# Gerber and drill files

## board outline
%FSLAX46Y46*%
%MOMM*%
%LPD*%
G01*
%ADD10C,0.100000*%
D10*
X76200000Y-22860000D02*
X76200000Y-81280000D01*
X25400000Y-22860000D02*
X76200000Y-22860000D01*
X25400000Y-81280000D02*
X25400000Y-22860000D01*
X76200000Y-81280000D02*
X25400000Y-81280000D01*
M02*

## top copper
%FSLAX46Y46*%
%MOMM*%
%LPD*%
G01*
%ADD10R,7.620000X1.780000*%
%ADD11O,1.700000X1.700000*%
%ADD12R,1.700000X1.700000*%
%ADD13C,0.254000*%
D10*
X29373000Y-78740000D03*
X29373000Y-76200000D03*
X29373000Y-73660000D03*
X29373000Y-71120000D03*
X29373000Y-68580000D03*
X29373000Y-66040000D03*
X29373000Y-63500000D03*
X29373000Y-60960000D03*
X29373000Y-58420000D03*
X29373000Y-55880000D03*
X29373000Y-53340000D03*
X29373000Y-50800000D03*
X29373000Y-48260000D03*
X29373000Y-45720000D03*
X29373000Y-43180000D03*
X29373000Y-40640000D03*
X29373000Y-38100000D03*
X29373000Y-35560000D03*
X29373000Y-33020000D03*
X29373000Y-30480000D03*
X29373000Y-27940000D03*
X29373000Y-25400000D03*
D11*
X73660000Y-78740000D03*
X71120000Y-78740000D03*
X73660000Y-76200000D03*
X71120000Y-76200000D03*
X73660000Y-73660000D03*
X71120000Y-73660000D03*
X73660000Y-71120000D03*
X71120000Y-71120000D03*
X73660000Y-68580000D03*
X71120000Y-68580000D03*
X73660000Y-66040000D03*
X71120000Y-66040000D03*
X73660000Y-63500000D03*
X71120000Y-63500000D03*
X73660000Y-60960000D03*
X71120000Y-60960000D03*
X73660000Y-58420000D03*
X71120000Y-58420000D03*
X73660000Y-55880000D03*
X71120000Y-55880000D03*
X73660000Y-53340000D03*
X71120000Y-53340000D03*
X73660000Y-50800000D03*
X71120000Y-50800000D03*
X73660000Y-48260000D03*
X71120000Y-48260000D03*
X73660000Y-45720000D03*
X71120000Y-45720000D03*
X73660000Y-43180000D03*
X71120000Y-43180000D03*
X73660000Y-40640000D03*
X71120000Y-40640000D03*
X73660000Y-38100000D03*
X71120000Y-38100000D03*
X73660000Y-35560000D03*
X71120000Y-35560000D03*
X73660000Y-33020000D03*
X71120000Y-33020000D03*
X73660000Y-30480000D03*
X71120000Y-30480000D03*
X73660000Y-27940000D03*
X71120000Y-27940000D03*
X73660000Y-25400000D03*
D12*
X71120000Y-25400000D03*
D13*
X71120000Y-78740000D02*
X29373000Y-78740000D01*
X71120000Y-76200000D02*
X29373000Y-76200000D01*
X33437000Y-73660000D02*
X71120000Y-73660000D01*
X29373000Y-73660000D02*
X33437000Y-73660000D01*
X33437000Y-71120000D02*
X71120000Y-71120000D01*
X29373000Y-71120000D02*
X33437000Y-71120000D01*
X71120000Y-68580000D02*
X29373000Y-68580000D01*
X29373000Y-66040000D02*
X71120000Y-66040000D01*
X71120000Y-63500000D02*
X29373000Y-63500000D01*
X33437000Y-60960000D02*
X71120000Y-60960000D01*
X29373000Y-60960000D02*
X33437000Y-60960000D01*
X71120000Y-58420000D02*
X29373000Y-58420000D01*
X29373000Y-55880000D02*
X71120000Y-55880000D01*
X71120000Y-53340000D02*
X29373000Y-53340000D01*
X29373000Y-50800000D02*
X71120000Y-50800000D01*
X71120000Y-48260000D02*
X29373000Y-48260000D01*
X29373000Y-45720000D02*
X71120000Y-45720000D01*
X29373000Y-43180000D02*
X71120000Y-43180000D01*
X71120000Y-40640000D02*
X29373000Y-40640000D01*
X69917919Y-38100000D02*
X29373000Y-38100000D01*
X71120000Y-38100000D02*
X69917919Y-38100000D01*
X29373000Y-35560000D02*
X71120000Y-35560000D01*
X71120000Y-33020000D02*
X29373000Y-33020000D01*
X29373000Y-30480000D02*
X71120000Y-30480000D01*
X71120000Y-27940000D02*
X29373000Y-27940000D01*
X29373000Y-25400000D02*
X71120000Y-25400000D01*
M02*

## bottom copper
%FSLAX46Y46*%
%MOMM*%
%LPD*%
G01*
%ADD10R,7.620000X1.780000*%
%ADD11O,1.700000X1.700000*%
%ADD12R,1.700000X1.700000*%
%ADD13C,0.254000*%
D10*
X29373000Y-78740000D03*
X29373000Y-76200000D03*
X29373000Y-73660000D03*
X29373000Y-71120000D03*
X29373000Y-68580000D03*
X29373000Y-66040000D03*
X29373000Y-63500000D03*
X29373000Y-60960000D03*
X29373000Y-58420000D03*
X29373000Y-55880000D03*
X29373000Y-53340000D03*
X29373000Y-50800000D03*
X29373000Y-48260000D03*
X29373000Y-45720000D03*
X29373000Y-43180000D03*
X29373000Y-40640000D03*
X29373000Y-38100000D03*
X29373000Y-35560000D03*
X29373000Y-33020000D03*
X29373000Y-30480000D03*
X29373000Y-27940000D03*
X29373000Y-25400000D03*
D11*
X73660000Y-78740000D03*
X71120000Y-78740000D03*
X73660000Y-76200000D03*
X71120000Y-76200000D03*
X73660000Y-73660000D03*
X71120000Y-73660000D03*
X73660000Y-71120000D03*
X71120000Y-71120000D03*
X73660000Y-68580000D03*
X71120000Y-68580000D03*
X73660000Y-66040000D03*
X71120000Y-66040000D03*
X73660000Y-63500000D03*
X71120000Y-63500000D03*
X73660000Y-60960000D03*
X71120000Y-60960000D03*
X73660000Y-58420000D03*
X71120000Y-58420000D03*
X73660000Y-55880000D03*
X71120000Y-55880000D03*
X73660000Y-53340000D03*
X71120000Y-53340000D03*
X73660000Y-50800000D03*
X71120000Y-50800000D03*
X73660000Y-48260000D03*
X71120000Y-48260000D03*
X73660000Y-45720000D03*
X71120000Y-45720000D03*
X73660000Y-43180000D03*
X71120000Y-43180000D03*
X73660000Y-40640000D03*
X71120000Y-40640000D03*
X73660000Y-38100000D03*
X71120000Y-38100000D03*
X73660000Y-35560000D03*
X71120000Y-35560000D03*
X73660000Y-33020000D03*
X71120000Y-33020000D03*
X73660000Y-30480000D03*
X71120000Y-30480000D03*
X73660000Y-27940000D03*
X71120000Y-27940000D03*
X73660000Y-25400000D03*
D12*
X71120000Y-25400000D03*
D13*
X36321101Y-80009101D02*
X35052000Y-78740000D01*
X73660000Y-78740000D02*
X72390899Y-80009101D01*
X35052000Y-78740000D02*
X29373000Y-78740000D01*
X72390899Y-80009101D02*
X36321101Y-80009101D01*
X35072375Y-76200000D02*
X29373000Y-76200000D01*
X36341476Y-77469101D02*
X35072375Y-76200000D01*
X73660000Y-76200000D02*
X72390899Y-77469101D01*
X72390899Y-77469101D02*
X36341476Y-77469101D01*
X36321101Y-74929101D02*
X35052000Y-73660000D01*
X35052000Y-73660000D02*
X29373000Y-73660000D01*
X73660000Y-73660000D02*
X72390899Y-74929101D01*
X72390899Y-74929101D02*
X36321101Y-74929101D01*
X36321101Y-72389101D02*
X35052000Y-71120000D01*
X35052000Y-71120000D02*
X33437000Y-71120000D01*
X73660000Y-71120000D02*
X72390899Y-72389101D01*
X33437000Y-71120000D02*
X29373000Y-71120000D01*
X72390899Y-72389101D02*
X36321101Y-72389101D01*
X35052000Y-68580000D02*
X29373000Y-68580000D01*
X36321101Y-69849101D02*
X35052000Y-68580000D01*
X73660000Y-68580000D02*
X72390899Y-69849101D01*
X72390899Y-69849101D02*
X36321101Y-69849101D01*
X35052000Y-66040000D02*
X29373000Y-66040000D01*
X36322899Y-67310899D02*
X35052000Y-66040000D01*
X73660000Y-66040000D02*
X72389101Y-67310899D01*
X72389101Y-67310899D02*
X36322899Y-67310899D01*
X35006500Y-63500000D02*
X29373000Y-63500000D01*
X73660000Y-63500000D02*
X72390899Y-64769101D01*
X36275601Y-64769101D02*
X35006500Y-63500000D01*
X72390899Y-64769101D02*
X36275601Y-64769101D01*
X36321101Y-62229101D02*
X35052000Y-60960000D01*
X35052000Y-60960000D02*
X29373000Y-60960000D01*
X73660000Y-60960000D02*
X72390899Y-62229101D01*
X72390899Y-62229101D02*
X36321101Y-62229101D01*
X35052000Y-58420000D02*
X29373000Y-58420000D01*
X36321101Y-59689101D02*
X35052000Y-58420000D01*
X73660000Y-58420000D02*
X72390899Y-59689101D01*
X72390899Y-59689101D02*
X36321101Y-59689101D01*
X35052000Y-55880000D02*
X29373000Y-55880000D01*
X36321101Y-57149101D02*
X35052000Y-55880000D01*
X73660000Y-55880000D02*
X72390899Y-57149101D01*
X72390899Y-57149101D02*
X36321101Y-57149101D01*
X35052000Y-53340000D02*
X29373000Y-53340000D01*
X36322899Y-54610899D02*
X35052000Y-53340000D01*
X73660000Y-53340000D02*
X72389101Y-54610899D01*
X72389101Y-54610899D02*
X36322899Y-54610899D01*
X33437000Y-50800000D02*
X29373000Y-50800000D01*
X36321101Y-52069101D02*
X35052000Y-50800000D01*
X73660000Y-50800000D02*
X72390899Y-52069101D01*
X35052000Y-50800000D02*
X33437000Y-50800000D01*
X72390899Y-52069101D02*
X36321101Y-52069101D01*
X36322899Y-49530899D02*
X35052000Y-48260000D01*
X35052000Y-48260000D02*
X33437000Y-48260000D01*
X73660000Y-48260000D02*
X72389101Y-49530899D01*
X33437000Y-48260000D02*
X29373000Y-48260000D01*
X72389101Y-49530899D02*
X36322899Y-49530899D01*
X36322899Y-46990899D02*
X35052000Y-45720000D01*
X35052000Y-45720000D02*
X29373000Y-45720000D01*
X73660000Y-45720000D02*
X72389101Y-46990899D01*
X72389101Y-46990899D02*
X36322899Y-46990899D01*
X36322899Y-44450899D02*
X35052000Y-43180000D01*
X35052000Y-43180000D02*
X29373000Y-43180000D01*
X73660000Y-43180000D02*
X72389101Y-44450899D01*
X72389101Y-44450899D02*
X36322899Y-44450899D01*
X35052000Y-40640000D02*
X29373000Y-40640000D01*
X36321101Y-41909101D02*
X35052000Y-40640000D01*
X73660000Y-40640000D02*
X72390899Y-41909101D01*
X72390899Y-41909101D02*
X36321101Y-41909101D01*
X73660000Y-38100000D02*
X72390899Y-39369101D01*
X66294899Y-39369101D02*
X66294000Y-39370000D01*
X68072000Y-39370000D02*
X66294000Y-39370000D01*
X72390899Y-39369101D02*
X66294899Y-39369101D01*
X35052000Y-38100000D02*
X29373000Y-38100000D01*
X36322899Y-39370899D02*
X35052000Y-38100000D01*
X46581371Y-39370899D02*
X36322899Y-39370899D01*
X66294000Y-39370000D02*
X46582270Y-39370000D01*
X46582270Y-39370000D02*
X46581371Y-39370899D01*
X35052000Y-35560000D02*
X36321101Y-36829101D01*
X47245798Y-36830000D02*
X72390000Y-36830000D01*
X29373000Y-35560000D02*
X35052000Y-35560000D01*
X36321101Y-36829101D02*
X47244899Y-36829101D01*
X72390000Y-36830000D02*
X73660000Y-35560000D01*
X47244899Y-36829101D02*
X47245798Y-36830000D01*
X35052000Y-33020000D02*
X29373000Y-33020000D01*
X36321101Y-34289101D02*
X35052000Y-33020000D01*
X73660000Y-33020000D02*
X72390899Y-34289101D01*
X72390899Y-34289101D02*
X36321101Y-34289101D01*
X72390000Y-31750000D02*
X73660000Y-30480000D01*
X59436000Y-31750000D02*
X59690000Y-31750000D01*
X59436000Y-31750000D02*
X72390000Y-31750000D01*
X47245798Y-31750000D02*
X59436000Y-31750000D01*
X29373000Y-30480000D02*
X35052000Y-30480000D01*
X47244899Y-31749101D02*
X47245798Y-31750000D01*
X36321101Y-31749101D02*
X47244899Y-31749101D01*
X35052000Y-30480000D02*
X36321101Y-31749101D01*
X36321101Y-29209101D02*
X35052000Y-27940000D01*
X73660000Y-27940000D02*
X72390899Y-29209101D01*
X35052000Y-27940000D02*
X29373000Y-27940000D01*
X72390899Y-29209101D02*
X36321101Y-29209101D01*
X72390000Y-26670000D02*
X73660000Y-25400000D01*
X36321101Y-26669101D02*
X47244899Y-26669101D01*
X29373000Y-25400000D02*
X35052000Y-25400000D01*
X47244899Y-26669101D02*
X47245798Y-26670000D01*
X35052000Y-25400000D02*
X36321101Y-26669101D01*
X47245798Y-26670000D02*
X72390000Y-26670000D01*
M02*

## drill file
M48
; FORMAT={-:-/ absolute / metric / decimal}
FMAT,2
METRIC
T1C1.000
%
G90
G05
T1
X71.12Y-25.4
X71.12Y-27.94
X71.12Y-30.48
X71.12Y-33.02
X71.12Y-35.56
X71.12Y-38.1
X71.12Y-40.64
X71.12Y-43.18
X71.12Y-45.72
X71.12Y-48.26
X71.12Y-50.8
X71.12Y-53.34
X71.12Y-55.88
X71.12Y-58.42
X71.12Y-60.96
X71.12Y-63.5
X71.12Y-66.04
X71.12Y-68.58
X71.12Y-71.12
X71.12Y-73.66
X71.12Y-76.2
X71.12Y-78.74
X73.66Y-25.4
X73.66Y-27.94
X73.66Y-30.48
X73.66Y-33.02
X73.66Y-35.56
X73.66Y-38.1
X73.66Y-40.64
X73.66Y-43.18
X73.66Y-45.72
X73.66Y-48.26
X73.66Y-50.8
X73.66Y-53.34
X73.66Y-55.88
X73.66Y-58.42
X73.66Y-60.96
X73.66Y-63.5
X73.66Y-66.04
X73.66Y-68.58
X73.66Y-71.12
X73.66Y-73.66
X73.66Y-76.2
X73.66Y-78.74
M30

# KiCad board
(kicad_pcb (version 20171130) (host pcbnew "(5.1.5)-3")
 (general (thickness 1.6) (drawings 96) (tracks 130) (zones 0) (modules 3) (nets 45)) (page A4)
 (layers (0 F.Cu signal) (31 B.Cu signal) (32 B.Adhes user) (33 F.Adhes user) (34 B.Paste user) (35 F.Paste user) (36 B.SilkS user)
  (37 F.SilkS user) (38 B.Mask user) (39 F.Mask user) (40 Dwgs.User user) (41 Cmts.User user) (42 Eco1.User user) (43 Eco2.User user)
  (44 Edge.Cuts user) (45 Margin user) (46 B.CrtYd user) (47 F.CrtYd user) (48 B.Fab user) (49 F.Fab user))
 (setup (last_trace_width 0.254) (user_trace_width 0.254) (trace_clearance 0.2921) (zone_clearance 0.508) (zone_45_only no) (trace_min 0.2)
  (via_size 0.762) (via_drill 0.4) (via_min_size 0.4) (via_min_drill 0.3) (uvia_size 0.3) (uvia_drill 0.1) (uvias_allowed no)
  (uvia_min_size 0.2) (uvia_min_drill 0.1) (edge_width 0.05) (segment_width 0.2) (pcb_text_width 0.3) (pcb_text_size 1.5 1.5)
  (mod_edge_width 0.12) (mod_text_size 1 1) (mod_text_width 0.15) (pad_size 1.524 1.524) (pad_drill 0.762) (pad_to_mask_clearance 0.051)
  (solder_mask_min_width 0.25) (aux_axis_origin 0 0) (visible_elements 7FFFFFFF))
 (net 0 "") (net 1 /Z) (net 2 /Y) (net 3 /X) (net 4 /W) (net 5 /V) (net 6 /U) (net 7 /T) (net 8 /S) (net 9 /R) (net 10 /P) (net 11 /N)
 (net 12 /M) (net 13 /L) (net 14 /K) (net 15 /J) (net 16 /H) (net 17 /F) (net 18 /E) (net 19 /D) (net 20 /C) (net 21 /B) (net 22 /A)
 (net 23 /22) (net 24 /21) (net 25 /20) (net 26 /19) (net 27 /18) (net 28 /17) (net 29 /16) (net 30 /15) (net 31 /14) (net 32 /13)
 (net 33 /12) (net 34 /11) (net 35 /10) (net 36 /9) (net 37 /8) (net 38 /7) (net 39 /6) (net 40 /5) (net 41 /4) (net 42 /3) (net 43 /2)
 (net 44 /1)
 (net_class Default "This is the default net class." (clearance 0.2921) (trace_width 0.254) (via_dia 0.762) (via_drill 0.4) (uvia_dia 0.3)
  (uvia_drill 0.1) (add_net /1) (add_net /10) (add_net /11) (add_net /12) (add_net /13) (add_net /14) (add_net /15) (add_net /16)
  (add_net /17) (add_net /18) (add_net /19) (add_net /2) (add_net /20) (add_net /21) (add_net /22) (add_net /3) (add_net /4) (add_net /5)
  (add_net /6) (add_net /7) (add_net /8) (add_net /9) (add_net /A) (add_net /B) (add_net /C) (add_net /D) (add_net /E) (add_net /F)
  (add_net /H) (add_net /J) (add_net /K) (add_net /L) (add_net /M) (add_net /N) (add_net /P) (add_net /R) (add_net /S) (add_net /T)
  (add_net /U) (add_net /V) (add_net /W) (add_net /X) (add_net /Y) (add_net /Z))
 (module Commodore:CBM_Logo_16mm (layer F.Cu) (at 54.61 52.07 90)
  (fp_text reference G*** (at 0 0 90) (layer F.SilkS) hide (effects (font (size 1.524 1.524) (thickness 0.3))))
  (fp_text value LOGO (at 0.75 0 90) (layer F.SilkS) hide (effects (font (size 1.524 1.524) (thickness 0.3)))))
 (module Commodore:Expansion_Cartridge (layer F.Cu) (at 25.527 23.749 90)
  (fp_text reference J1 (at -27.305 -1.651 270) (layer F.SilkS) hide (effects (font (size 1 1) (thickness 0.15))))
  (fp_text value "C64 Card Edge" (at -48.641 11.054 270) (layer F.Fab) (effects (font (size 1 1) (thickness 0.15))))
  (pad Z connect rect (at -54.991 3.846 270) (size 1.78 7.62) (layers B.Cu B.Mask) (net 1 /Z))
  (pad Y connect rect (at -52.451 3.846 270) (size 1.78 7.62) (layers B.Cu B.Mask) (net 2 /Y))
  (pad X connect rect (at -49.911 3.846 270) (size 1.78 7.62) (layers B.Cu B.Mask) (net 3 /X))
  (pad W connect rect (at -47.371 3.846 270) (size 1.78 7.62) (layers B.Cu B.Mask) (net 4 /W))
  (pad V connect rect (at -44.831 3.846 270) (size 1.78 7.62) (layers B.Cu B.Mask) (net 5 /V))
  (pad U connect rect (at -42.291 3.846 270) (size 1.78 7.62) (layers B.Cu B.Mask) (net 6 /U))
  (pad T connect rect (at -39.751 3.846 270) (size 1.78 7.62) (layers B.Cu B.Mask) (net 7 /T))
  (pad S connect rect (at -37.211 3.846 270) (size 1.78 7.62) (layers B.Cu B.Mask) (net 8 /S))
  (pad R connect rect (at -34.671 3.846 270) (size 1.78 7.62) (layers B.Cu B.Mask) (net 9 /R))
  (pad P connect rect (at -32.131 3.846 270) (size 1.78 7.62) (layers B.Cu B.Mask) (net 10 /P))
  (pad N connect rect (at -29.591 3.846 270) (size 1.78 7.62) (layers B.Cu B.Mask) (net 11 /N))
  (pad M connect rect (at -27.051 3.846 270) (size 1.78 7.62) (layers B.Cu B.Mask) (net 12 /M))
  (pad L connect rect (at -24.511 3.846 270) (size 1.78 7.62) (layers B.Cu B.Mask) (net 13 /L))
  (pad K connect rect (at -21.971 3.846 270) (size 1.78 7.62) (layers B.Cu B.Mask) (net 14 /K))
  (pad J connect rect (at -19.431 3.846 270) (size 1.78 7.62) (layers B.Cu B.Mask) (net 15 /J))
  (pad H connect rect (at -16.891 3.846 270) (size 1.78 7.62) (layers B.Cu B.Mask) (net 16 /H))
  (pad F connect rect (at -14.351 3.846 270) (size 1.78 7.62) (layers B.Cu B.Mask) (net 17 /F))
  (pad E connect rect (at -11.811 3.846 270) (size 1.78 7.62) (layers B.Cu B.Mask) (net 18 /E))
  (pad D connect rect (at -9.271 3.846 270) (size 1.78 7.62) (layers B.Cu B.Mask) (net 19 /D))
  (pad C connect rect (at -6.731 3.846 270) (size 1.78 7.62) (layers B.Cu B.Mask) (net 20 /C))
  (pad B connect rect (at -4.191 3.846 270) (size 1.78 7.62) (layers B.Cu B.Mask) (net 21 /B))
  (pad A connect rect (at -1.651 3.846 270) (size 1.78 7.62) (layers B.Cu B.Mask) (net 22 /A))
  (pad 22 connect rect (at -54.991 3.846 270) (size 1.78 7.62) (layers F.Cu F.Mask) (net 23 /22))
  (pad 21 connect rect (at -52.451 3.846 270) (size 1.78 7.62) (layers F.Cu F.Mask) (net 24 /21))
  (pad 20 connect rect (at -49.911 3.846 270) (size 1.78 7.62) (layers F.Cu F.Mask) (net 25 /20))
  (pad 19 connect rect (at -47.371 3.846 270) (size 1.78 7.62) (layers F.Cu F.Mask) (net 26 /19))
  (pad 18 connect rect (at -44.831 3.846 270) (size 1.78 7.62) (layers F.Cu F.Mask) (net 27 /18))
  (pad 17 connect rect (at -42.291 3.846 270) (size 1.78 7.62) (layers F.Cu F.Mask) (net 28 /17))
  (pad 16 connect rect (at -39.751 3.846 270) (size 1.78 7.62) (layers F.Cu F.Mask) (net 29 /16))
  (pad 15 connect rect (at -37.211 3.846 270) (size 1.78 7.62) (layers F.Cu F.Mask) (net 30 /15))
  (pad 14 connect rect (at -34.671 3.846 270) (size 1.78 7.62) (layers F.Cu F.Mask) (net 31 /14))
  (pad 13 connect rect (at -32.131 3.846 270) (size 1.78 7.62) (layers F.Cu F.Mask) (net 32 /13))
  (pad 12 connect rect (at -29.591 3.846 270) (size 1.78 7.62) (layers F.Cu F.Mask) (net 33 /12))
  (pad 11 connect rect (at -27.051 3.846 270) (size 1.78 7.62) (layers F.Cu F.Mask) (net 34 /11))
  (pad 10 connect rect (at -24.511 3.846 270) (size 1.78 7.62) (layers F.Cu F.Mask) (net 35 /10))
  (pad 9 connect rect (at -21.971 3.846 270) (size 1.78 7.62) (layers F.Cu F.Mask) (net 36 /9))
  (pad 8 connect rect (at -19.431 3.846 270) (size 1.78 7.62) (layers F.Cu F.Mask) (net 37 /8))
  (pad 7 connect rect (at -16.891 3.846 270) (size 1.78 7.62) (layers F.Cu F.Mask) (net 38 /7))
  (pad 6 connect rect (at -14.351 3.846 270) (size 1.78 7.62) (layers F.Cu F.Mask) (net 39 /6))
  (pad 5 connect rect (at -11.811 3.846 270) (size 1.78 7.62) (layers F.Cu F.Mask) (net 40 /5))
  (pad 4 connect rect (at -9.271 3.846 270) (size 1.78 7.62) (layers F.Cu F.Mask) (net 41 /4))
  (pad 3 connect rect (at -6.731 3.846 270) (size 1.78 7.62) (layers F.Cu F.Mask) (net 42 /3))
  (pad 2 connect rect (at -4.191 3.846 270) (size 1.78 7.62) (layers F.Cu F.Mask) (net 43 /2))
  (pad 1 connect rect (at -1.651 3.846 270) (size 1.78 7.62) (layers F.Cu F.Mask) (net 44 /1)))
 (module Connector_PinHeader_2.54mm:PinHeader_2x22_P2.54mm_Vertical (layer F.Cu) (at 71.12 25.4)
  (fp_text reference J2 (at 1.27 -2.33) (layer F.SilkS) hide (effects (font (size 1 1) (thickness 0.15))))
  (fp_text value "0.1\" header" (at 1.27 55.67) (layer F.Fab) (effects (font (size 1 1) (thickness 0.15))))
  (pad 44 thru_hole oval (at 2.54 53.34) (size 1.7 1.7) (drill 1) (layers *.Cu *.Mask) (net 1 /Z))
  (pad 43 thru_hole oval (at 0 53.34) (size 1.7 1.7) (drill 1) (layers *.Cu *.Mask) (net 23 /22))
  (pad 42 thru_hole oval (at 2.54 50.8) (size 1.7 1.7) (drill 1) (layers *.Cu *.Mask) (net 2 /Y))
  (pad 41 thru_hole oval (at 0 50.8) (size 1.7 1.7) (drill 1) (layers *.Cu *.Mask) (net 24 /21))
  (pad 40 thru_hole oval (at 2.54 48.26) (size 1.7 1.7) (drill 1) (layers *.Cu *.Mask) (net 3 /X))
  (pad 39 thru_hole oval (at 0 48.26) (size 1.7 1.7) (drill 1) (layers *.Cu *.Mask) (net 25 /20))
  (pad 38 thru_hole oval (at 2.54 45.72) (size 1.7 1.7) (drill 1) (layers *.Cu *.Mask) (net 4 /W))
  (pad 37 thru_hole oval (at 0 45.72) (size 1.7 1.7) (drill 1) (layers *.Cu *.Mask) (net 26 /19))
  (pad 36 thru_hole oval (at 2.54 43.18) (size 1.7 1.7) (drill 1) (layers *.Cu *.Mask) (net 5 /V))
  (pad 35 thru_hole oval (at 0 43.18) (size 1.7 1.7) (drill 1) (layers *.Cu *.Mask) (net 27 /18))
  (pad 34 thru_hole oval (at 2.54 40.64) (size 1.7 1.7) (drill 1) (layers *.Cu *.Mask) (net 6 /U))
  (pad 33 thru_hole oval (at 0 40.64) (size 1.7 1.7) (drill 1) (layers *.Cu *.Mask) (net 28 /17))
  (pad 32 thru_hole oval (at 2.54 38.1) (size 1.7 1.7) (drill 1) (layers *.Cu *.Mask) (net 7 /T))
  (pad 31 thru_hole oval (at 0 38.1) (size 1.7 1.7) (drill 1) (layers *.Cu *.Mask) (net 29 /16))
  (pad 30 thru_hole oval (at 2.54 35.56) (size 1.7 1.7) (drill 1) (layers *.Cu *.Mask) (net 8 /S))
  (pad 29 thru_hole oval (at 0 35.56) (size 1.7 1.7) (drill 1) (layers *.Cu *.Mask) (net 30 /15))
  (pad 28 thru_hole oval (at 2.54 33.02) (size 1.7 1.7) (drill 1) (layers *.Cu *.Mask) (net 9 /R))
  (pad 27 thru_hole oval (at 0 33.02) (size 1.7 1.7) (drill 1) (layers *.Cu *.Mask) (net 31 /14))
  (pad 26 thru_hole oval (at 2.54 30.48) (size 1.7 1.7) (drill 1) (layers *.Cu *.Mask) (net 10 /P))
  (pad 25 thru_hole oval (at 0 30.48) (size 1.7 1.7) (drill 1) (layers *.Cu *.Mask) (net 32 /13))
  (pad 24 thru_hole oval (at 2.54 27.94) (size 1.7 1.7) (drill 1) (layers *.Cu *.Mask) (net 11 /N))
  (pad 23 thru_hole oval (at 0 27.94) (size 1.7 1.7) (drill 1) (layers *.Cu *.Mask) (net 33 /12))
  (pad 22 thru_hole oval (at 2.54 25.4) (size 1.7 1.7) (drill 1) (layers *.Cu *.Mask) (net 12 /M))
  (pad 21 thru_hole oval (at 0 25.4) (size 1.7 1.7) (drill 1) (layers *.Cu *.Mask) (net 34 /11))
  (pad 20 thru_hole oval (at 2.54 22.86) (size 1.7 1.7) (drill 1) (layers *.Cu *.Mask) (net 13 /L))
  (pad 19 thru_hole oval (at 0 22.86) (size 1.7 1.7) (drill 1) (layers *.Cu *.Mask) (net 35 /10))
  (pad 18 thru_hole oval (at 2.54 20.32) (size 1.7 1.7) (drill 1) (layers *.Cu *.Mask) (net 14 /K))
  (pad 17 thru_hole oval (at 0 20.32) (size 1.7 1.7) (drill 1) (layers *.Cu *.Mask) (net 36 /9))
  (pad 16 thru_hole oval (at 2.54 17.78) (size 1.7 1.7) (drill 1) (layers *.Cu *.Mask) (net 15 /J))
  (pad 15 thru_hole oval (at 0 17.78) (size 1.7 1.7) (drill 1) (layers *.Cu *.Mask) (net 37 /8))
  (pad 14 thru_hole oval (at 2.54 15.24) (size 1.7 1.7) (drill 1) (layers *.Cu *.Mask) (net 16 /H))
  (pad 13 thru_hole oval (at 0 15.24) (size 1.7 1.7) (drill 1) (layers *.Cu *.Mask) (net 38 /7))
  (pad 12 thru_hole oval (at 2.54 12.7) (size 1.7 1.7) (drill 1) (layers *.Cu *.Mask) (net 17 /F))
  (pad 11 thru_hole oval (at 0 12.7) (size 1.7 1.7) (drill 1) (layers *.Cu *.Mask) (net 39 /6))
  (pad 10 thru_hole oval (at 2.54 10.16) (size 1.7 1.7) (drill 1) (layers *.Cu *.Mask) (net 18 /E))
  (pad 9 thru_hole oval (at 0 10.16) (size 1.7 1.7) (drill 1) (layers *.Cu *.Mask) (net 40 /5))
  (pad 8 thru_hole oval (at 2.54 7.62) (size 1.7 1.7) (drill 1) (layers *.Cu *.Mask) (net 19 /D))
  (pad 7 thru_hole oval (at 0 7.62) (size 1.7 1.7) (drill 1) (layers *.Cu *.Mask) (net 41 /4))
  (pad 6 thru_hole oval (at 2.54 5.08) (size 1.7 1.7) (drill 1) (layers *.Cu *.Mask) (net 20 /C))
  (pad 5 thru_hole oval (at 0 5.08) (size 1.7 1.7) (drill 1) (layers *.Cu *.Mask) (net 42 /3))
  (pad 4 thru_hole oval (at 2.54 2.54) (size 1.7 1.7) (drill 1) (layers *.Cu *.Mask) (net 21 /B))
  (pad 3 thru_hole oval (at 0 2.54) (size 1.7 1.7) (drill 1) (layers *.Cu *.Mask) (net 43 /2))
  (pad 2 thru_hole oval (at 2.54 0) (size 1.7 1.7) (drill 1) (layers *.Cu *.Mask) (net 22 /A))
  (pad 1 thru_hole rect (at 0 0) (size 1.7 1.7) (drill 1) (layers *.Cu *.Mask) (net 44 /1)))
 (gr_line (start 76.2 22.86) (end 76.2 81.28) (layer Edge.Cuts) (width 0.1))
 (gr_line (start 25.4 22.86) (end 76.2 22.86) (layer Edge.Cuts) (width 0.1))
 (gr_line (start 25.4 81.28) (end 25.4 22.86) (layer Edge.Cuts) (width 0.1))
 (gr_line (start 76.2 81.28) (end 25.4 81.28) (layer Edge.Cuts) (width 0.1))
 (segment (start 71.12 78.74) (end 29.373 78.74) (width 0.254) (layer F.Cu) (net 23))
 (segment (start 71.12 76.2) (end 29.373 76.2) (width 0.254) (layer F.Cu) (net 24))
 (segment (start 33.437 73.66) (end 71.12 73.66) (width 0.254) (layer F.Cu) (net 25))
 (segment (start 29.373 73.66) (end 33.437 73.66) (width 0.254) (layer F.Cu) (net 25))
 (segment (start 33.437 71.12) (end 71.12 71.12) (width 0.254) (layer F.Cu) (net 26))
 (segment (start 29.373 71.12) (end 33.437 71.12) (width 0.254) (layer F.Cu) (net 26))
 (segment (start 71.12 68.58) (end 29.373 68.58) (width 0.254) (layer F.Cu) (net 27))
 (segment (start 29.373 66.04) (end 71.12 66.04) (width 0.254) (layer F.Cu) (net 28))
 (segment (start 71.12 63.5) (end 29.373 63.5) (width 0.254) (layer F.Cu) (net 29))
 (segment (start 33.437 60.96) (end 71.12 60.96) (width 0.254) (layer F.Cu) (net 30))
 (segment (start 29.373 60.96) (end 33.437 60.96) (width 0.254) (layer F.Cu) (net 30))
 (segment (start 71.12 58.42) (end 29.373 58.42) (width 0.254) (layer F.Cu) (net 31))
 (segment (start 29.373 55.88) (end 71.12 55.88) (width 0.254) (layer F.Cu) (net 32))
 (segment (start 71.12 53.34) (end 29.373 53.34) (width 0.254) (layer F.Cu) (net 33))
 (segment (start 29.373 50.8) (end 71.12 50.8) (width 0.254) (layer F.Cu) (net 34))
 (segment (start 71.12 48.26) (end 29.373 48.26) (width 0.254) (layer F.Cu) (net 35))
 (segment (start 29.373 45.72) (end 71.12 45.72) (width 0.254) (layer F.Cu) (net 36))
 (segment (start 29.373 43.18) (end 71.12 43.18) (width 0.254) (layer F.Cu) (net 37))
 (segment (start 71.12 40.64) (end 29.373 40.64) (width 0.254) (layer F.Cu) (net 38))
 (segment (start 69.917919 38.1) (end 29.373 38.1) (width 0.254) (layer F.Cu) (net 39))
 (segment (start 71.12 38.1) (end 69.917919 38.1) (width 0.254) (layer F.Cu) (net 39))
 (segment (start 29.373 35.56) (end 71.12 35.56) (width 0.254) (layer F.Cu) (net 40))
 (segment (start 71.12 33.02) (end 29.373 33.02) (width 0.254) (layer F.Cu) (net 41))
 (segment (start 29.373 30.48) (end 71.12 30.48) (width 0.254) (layer F.Cu) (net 42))
 (segment (start 71.12 27.94) (end 29.373 27.94) (width 0.254) (layer F.Cu) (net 43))
 (segment (start 29.373 25.4) (end 71.12 25.4) (width 0.254) (layer F.Cu) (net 44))
 (segment (start 36.321101 80.009101) (end 35.052 78.74) (width 0.254) (layer B.Cu) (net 1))
 (segment (start 73.66 78.74) (end 72.390899 80.009101) (width 0.254) (layer B.Cu) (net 1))
 (segment (start 35.052 78.74) (end 29.373 78.74) (width 0.254) (layer B.Cu) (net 1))
 (segment (start 72.390899 80.009101) (end 36.321101 80.009101) (width 0.254) (layer B.Cu) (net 1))
 (segment (start 35.072375 76.2) (end 29.373 76.2) (width 0.254) (layer B.Cu) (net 2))
 (segment (start 36.341476 77.469101) (end 35.072375 76.2) (width 0.254) (layer B.Cu) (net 2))
 (segment (start 73.66 76.2) (end 72.390899 77.469101) (width 0.254) (layer B.Cu) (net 2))
 (segment (start 72.390899 77.469101) (end 36.341476 77.469101) (width 0.254) (layer B.Cu) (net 2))
 (segment (start 36.321101 74.929101) (end 35.052 73.66) (width 0.254) (layer B.Cu) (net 3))
 (segment (start 35.052 73.66) (end 29.373 73.66) (width 0.254) (layer B.Cu) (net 3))
 (segment (start 73.66 73.66) (end 72.390899 74.929101) (width 0.254) (layer B.Cu) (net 3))
 (segment (start 72.390899 74.929101) (end 36.321101 74.929101) (width 0.254) (layer B.Cu) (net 3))
 (segment (start 36.321101 72.389101) (end 35.052 71.12) (width 0.254) (layer B.Cu) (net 4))
 (segment (start 35.052 71.12) (end 33.437 71.12) (width 0.254) (layer B.Cu) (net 4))
 (segment (start 73.66 71.12) (end 72.390899 72.389101) (width 0.254) (layer B.Cu) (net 4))
 (segment (start 33.437 71.12) (end 29.373 71.12) (width 0.254) (layer B.Cu) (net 4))
 (segment (start 72.390899 72.389101) (end 36.321101 72.389101) (width 0.254) (layer B.Cu) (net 4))
 (segment (start 35.052 68.58) (end 29.373 68.58) (width 0.254) (layer B.Cu) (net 5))
 (segment (start 36.321101 69.849101) (end 35.052 68.58) (width 0.254) (layer B.Cu) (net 5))
 (segment (start 73.66 68.58) (end 72.390899 69.849101) (width 0.254) (layer B.Cu) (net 5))
 (segment (start 72.390899 69.849101) (end 36.321101 69.849101) (width 0.254) (layer B.Cu) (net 5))
 (segment (start 35.052 66.04) (end 29.373 66.04) (width 0.254) (layer B.Cu) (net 6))
 (segment (start 36.322899 67.310899) (end 35.052 66.04) (width 0.254) (layer B.Cu) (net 6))
 (segment (start 73.66 66.04) (end 72.389101 67.310899) (width 0.254) (layer B.Cu) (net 6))
 (segment (start 72.389101 67.310899) (end 36.322899 67.310899) (width 0.254) (layer B.Cu) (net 6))
 (segment (start 35.0065 63.5) (end 29.373 63.5) (width 0.254) (layer B.Cu) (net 7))
 (segment (start 73.66 63.5) (end 72.390899 64.769101) (width 0.254) (layer B.Cu) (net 7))
 (segment (start 36.275601 64.769101) (end 35.0065 63.5) (width 0.254) (layer B.Cu) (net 7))
 (segment (start 72.390899 64.769101) (end 36.275601 64.769101) (width 0.254) (layer B.Cu) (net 7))
 (segment (start 36.321101 62.229101) (end 35.052 60.96) (width 0.254) (layer B.Cu) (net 8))
 (segment (start 35.052 60.96) (end 29.373 60.96) (width 0.254) (layer B.Cu) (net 8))
 (segment (start 73.66 60.96) (end 72.390899 62.229101) (width 0.254) (layer B.Cu) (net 8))
 (segment (start 72.390899 62.229101) (end 36.321101 62.229101) (width 0.254) (layer B.Cu) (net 8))
 (segment (start 35.052 58.42) (end 29.373 58.42) (width 0.254) (layer B.Cu) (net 9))
 (segment (start 36.321101 59.689101) (end 35.052 58.42) (width 0.254) (layer B.Cu) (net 9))
 (segment (start 73.66 58.42) (end 72.390899 59.689101) (width 0.254) (layer B.Cu) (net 9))
 (segment (start 72.390899 59.689101) (end 36.321101 59.689101) (width 0.254) (layer B.Cu) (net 9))
 (segment (start 35.052 55.88) (end 29.373 55.88) (width 0.254) (layer B.Cu) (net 10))
 (segment (start 36.321101 57.149101) (end 35.052 55.88) (width 0.254) (layer B.Cu) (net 10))
 (segment (start 73.66 55.88) (end 72.390899 57.149101) (width 0.254) (layer B.Cu) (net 10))
 (segment (start 72.390899 57.149101) (end 36.321101 57.149101) (width 0.254) (layer B.Cu) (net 10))
 (segment (start 35.052 53.34) (end 29.373 53.34) (width 0.254) (layer B.Cu) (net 11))
 (segment (start 36.322899 54.610899) (end 35.052 53.34) (width 0.254) (layer B.Cu) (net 11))
 (segment (start 73.66 53.34) (end 72.389101 54.610899) (width 0.254) (layer B.Cu) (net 11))
 (segment (start 72.389101 54.610899) (end 36.322899 54.610899) (width 0.254) (layer B.Cu) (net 11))
 (segment (start 33.437 50.8) (end 29.373 50.8) (width 0.254) (layer B.Cu) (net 12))
 (segment (start 36.321101 52.069101) (end 35.052 50.8) (width 0.254) (layer B.Cu) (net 12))
 (segment (start 73.66 50.8) (end 72.390899 52.069101) (width 0.254) (layer B.Cu) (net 12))
 (segment (start 35.052 50.8) (end 33.437 50.8) (width 0.254) (layer B.Cu) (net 12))
 (segment (start 72.390899 52.069101) (end 36.321101 52.069101) (width 0.254) (layer B.Cu) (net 12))
 (segment (start 36.322899 49.530899) (end 35.052 48.26) (width 0.254) (layer B.Cu) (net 13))
 (segment (start 35.052 48.26) (end 33.437 48.26) (width 0.254) (layer B.Cu) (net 13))
 (segment (start 73.66 48.26) (end 72.389101 49.530899) (width 0.254) (layer B.Cu) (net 13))
 (segment (start 33.437 48.26) (end 29.373 48.26) (width 0.254) (layer B.Cu) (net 13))
 (segment (start 72.389101 49.530899) (end 36.322899 49.530899) (width 0.254) (layer B.Cu) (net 13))
 (segment (start 36.322899 46.990899) (end 35.052 45.72) (width 0.254) (layer B.Cu) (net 14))
 (segment (start 35.052 45.72) (end 29.373 45.72) (width 0.254) (layer B.Cu) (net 14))
 (segment (start 73.66 45.72) (end 72.389101 46.990899) (width 0.254) (layer B.Cu) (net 14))
 (segment (start 72.389101 46.990899) (end 36.322899 46.990899) (width 0.254) (layer B.Cu) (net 14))
 (segment (start 36.322899 44.450899) (end 35.052 43.18) (width 0.254) (layer B.Cu) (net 15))
 (segment (start 35.052 43.18) (end 29.373 43.18) (width 0.254) (layer B.Cu) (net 15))
 (segment (start 73.66 43.18) (end 72.389101 44.450899) (width 0.254) (layer B.Cu) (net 15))
 (segment (start 72.389101 44.450899) (end 36.322899 44.450899) (width 0.254) (layer B.Cu) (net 15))
 (segment (start 35.052 40.64) (end 29.373 40.64) (width 0.254) (layer B.Cu) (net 16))
 (segment (start 36.321101 41.909101) (end 35.052 40.64) (width 0.254) (layer B.Cu) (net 16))
 (segment (start 73.66 40.64) (end 72.390899 41.909101) (width 0.254) (layer B.Cu) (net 16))
 (segment (start 72.390899 41.909101) (end 36.321101 41.909101) (width 0.254) (layer B.Cu) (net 16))
 (segment (start 73.66 38.1) (end 72.390899 39.369101) (width 0.254) (layer B.Cu) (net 17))
 (segment (start 66.294899 39.369101) (end 66.294 39.37) (width 0.254) (layer B.Cu) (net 17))
 (segment (start 68.072 39.37) (end 66.294 39.37) (width 0.254) (layer B.Cu) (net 17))
 (segment (start 72.390899 39.369101) (end 66.294899 39.369101) (width 0.254) (layer B.Cu) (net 17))
 (segment (start 35.052 38.1) (end 29.373 38.1) (width 0.254) (layer B.Cu) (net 17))
 (segment (start 36.322899 39.370899) (end 35.052 38.1) (width 0.254) (layer B.Cu) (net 17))
 (segment (start 46.581371 39.370899) (end 36.322899 39.370899) (width 0.254) (layer B.Cu) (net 17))
 (segment (start 66.294 39.37) (end 46.58227 39.37) (width 0.254) (layer B.Cu) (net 17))
 (segment (start 46.58227 39.37) (end 46.581371 39.370899) (width 0.254) (layer B.Cu) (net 17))
 (segment (start 35.052 35.56) (end 36.321101 36.829101) (width 0.254) (layer B.Cu) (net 18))
 (segment (start 47.245798 36.83) (end 72.39 36.83) (width 0.254) (layer B.Cu) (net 18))
 (segment (start 29.373 35.56) (end 35.052 35.56) (width 0.254) (layer B.Cu) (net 18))
 (segment (start 36.321101 36.829101) (end 47.244899 36.829101) (width 0.254) (layer B.Cu) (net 18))
 (segment (start 72.39 36.83) (end 73.66 35.56) (width 0.254) (layer B.Cu) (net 18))
 (segment (start 47.244899 36.829101) (end 47.245798 36.83) (width 0.254) (layer B.Cu) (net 18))
 (segment (start 35.052 33.02) (end 29.373 33.02) (width 0.254) (layer B.Cu) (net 19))
 (segment (start 36.321101 34.289101) (end 35.052 33.02) (width 0.254) (layer B.Cu) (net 19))
 (segment (start 73.66 33.02) (end 72.390899 34.289101) (width 0.254) (layer B.Cu) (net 19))
 (segment (start 72.390899 34.289101) (end 36.321101 34.289101) (width 0.254) (layer B.Cu) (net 19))
 (segment (start 72.39 31.75) (end 73.66 30.48) (width 0.254) (layer B.Cu) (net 20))
 (segment (start 59.436 31.75) (end 59.69 31.75) (width 0.254) (layer B.Cu) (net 20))
 (segment (start 59.436 31.75) (end 72.39 31.75) (width 0.254) (layer B.Cu) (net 20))
 (segment (start 47.245798 31.75) (end 59.436 31.75) (width 0.254) (layer B.Cu) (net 20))
 (segment (start 29.373 30.48) (end 35.052 30.48) (width 0.254) (layer B.Cu) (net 20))
 (segment (start 47.244899 31.749101) (end 47.245798 31.75) (width 0.254) (layer B.Cu) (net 20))
 (segment (start 36.321101 31.749101) (end 47.244899 31.749101) (width 0.254) (layer B.Cu) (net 20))
 (segment (start 35.052 30.48) (end 36.321101 31.749101) (width 0.254) (layer B.Cu) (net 20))
 (segment (start 36.321101 29.209101) (end 35.052 27.94) (width 0.254) (layer B.Cu) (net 21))
 (segment (start 73.66 27.94) (end 72.390899 29.209101) (width 0.254) (layer B.Cu) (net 21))
 (segment (start 35.052 27.94) (end 29.373 27.94) (width 0.254) (layer B.Cu) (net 21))
 (segment (start 72.390899 29.209101) (end 36.321101 29.209101) (width 0.254) (layer B.Cu) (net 21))
 (segment (start 72.39 26.67) (end 73.66 25.4) (width 0.254) (layer B.Cu) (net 22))
 (segment (start 36.321101 26.669101) (end 47.244899 26.669101) (width 0.254) (layer B.Cu) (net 22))
 (segment (start 29.373 25.4) (end 35.052 25.4) (width 0.254) (layer B.Cu) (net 22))
 (segment (start 47.244899 26.669101) (end 47.245798 26.67) (width 0.254) (layer B.Cu) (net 22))
 (segment (start 35.052 25.4) (end 36.321101 26.669101) (width 0.254) (layer B.Cu) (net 22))
 (segment (start 47.245798 26.67) (end 72.39 26.67) (width 0.254) (layer B.Cu) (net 22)))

